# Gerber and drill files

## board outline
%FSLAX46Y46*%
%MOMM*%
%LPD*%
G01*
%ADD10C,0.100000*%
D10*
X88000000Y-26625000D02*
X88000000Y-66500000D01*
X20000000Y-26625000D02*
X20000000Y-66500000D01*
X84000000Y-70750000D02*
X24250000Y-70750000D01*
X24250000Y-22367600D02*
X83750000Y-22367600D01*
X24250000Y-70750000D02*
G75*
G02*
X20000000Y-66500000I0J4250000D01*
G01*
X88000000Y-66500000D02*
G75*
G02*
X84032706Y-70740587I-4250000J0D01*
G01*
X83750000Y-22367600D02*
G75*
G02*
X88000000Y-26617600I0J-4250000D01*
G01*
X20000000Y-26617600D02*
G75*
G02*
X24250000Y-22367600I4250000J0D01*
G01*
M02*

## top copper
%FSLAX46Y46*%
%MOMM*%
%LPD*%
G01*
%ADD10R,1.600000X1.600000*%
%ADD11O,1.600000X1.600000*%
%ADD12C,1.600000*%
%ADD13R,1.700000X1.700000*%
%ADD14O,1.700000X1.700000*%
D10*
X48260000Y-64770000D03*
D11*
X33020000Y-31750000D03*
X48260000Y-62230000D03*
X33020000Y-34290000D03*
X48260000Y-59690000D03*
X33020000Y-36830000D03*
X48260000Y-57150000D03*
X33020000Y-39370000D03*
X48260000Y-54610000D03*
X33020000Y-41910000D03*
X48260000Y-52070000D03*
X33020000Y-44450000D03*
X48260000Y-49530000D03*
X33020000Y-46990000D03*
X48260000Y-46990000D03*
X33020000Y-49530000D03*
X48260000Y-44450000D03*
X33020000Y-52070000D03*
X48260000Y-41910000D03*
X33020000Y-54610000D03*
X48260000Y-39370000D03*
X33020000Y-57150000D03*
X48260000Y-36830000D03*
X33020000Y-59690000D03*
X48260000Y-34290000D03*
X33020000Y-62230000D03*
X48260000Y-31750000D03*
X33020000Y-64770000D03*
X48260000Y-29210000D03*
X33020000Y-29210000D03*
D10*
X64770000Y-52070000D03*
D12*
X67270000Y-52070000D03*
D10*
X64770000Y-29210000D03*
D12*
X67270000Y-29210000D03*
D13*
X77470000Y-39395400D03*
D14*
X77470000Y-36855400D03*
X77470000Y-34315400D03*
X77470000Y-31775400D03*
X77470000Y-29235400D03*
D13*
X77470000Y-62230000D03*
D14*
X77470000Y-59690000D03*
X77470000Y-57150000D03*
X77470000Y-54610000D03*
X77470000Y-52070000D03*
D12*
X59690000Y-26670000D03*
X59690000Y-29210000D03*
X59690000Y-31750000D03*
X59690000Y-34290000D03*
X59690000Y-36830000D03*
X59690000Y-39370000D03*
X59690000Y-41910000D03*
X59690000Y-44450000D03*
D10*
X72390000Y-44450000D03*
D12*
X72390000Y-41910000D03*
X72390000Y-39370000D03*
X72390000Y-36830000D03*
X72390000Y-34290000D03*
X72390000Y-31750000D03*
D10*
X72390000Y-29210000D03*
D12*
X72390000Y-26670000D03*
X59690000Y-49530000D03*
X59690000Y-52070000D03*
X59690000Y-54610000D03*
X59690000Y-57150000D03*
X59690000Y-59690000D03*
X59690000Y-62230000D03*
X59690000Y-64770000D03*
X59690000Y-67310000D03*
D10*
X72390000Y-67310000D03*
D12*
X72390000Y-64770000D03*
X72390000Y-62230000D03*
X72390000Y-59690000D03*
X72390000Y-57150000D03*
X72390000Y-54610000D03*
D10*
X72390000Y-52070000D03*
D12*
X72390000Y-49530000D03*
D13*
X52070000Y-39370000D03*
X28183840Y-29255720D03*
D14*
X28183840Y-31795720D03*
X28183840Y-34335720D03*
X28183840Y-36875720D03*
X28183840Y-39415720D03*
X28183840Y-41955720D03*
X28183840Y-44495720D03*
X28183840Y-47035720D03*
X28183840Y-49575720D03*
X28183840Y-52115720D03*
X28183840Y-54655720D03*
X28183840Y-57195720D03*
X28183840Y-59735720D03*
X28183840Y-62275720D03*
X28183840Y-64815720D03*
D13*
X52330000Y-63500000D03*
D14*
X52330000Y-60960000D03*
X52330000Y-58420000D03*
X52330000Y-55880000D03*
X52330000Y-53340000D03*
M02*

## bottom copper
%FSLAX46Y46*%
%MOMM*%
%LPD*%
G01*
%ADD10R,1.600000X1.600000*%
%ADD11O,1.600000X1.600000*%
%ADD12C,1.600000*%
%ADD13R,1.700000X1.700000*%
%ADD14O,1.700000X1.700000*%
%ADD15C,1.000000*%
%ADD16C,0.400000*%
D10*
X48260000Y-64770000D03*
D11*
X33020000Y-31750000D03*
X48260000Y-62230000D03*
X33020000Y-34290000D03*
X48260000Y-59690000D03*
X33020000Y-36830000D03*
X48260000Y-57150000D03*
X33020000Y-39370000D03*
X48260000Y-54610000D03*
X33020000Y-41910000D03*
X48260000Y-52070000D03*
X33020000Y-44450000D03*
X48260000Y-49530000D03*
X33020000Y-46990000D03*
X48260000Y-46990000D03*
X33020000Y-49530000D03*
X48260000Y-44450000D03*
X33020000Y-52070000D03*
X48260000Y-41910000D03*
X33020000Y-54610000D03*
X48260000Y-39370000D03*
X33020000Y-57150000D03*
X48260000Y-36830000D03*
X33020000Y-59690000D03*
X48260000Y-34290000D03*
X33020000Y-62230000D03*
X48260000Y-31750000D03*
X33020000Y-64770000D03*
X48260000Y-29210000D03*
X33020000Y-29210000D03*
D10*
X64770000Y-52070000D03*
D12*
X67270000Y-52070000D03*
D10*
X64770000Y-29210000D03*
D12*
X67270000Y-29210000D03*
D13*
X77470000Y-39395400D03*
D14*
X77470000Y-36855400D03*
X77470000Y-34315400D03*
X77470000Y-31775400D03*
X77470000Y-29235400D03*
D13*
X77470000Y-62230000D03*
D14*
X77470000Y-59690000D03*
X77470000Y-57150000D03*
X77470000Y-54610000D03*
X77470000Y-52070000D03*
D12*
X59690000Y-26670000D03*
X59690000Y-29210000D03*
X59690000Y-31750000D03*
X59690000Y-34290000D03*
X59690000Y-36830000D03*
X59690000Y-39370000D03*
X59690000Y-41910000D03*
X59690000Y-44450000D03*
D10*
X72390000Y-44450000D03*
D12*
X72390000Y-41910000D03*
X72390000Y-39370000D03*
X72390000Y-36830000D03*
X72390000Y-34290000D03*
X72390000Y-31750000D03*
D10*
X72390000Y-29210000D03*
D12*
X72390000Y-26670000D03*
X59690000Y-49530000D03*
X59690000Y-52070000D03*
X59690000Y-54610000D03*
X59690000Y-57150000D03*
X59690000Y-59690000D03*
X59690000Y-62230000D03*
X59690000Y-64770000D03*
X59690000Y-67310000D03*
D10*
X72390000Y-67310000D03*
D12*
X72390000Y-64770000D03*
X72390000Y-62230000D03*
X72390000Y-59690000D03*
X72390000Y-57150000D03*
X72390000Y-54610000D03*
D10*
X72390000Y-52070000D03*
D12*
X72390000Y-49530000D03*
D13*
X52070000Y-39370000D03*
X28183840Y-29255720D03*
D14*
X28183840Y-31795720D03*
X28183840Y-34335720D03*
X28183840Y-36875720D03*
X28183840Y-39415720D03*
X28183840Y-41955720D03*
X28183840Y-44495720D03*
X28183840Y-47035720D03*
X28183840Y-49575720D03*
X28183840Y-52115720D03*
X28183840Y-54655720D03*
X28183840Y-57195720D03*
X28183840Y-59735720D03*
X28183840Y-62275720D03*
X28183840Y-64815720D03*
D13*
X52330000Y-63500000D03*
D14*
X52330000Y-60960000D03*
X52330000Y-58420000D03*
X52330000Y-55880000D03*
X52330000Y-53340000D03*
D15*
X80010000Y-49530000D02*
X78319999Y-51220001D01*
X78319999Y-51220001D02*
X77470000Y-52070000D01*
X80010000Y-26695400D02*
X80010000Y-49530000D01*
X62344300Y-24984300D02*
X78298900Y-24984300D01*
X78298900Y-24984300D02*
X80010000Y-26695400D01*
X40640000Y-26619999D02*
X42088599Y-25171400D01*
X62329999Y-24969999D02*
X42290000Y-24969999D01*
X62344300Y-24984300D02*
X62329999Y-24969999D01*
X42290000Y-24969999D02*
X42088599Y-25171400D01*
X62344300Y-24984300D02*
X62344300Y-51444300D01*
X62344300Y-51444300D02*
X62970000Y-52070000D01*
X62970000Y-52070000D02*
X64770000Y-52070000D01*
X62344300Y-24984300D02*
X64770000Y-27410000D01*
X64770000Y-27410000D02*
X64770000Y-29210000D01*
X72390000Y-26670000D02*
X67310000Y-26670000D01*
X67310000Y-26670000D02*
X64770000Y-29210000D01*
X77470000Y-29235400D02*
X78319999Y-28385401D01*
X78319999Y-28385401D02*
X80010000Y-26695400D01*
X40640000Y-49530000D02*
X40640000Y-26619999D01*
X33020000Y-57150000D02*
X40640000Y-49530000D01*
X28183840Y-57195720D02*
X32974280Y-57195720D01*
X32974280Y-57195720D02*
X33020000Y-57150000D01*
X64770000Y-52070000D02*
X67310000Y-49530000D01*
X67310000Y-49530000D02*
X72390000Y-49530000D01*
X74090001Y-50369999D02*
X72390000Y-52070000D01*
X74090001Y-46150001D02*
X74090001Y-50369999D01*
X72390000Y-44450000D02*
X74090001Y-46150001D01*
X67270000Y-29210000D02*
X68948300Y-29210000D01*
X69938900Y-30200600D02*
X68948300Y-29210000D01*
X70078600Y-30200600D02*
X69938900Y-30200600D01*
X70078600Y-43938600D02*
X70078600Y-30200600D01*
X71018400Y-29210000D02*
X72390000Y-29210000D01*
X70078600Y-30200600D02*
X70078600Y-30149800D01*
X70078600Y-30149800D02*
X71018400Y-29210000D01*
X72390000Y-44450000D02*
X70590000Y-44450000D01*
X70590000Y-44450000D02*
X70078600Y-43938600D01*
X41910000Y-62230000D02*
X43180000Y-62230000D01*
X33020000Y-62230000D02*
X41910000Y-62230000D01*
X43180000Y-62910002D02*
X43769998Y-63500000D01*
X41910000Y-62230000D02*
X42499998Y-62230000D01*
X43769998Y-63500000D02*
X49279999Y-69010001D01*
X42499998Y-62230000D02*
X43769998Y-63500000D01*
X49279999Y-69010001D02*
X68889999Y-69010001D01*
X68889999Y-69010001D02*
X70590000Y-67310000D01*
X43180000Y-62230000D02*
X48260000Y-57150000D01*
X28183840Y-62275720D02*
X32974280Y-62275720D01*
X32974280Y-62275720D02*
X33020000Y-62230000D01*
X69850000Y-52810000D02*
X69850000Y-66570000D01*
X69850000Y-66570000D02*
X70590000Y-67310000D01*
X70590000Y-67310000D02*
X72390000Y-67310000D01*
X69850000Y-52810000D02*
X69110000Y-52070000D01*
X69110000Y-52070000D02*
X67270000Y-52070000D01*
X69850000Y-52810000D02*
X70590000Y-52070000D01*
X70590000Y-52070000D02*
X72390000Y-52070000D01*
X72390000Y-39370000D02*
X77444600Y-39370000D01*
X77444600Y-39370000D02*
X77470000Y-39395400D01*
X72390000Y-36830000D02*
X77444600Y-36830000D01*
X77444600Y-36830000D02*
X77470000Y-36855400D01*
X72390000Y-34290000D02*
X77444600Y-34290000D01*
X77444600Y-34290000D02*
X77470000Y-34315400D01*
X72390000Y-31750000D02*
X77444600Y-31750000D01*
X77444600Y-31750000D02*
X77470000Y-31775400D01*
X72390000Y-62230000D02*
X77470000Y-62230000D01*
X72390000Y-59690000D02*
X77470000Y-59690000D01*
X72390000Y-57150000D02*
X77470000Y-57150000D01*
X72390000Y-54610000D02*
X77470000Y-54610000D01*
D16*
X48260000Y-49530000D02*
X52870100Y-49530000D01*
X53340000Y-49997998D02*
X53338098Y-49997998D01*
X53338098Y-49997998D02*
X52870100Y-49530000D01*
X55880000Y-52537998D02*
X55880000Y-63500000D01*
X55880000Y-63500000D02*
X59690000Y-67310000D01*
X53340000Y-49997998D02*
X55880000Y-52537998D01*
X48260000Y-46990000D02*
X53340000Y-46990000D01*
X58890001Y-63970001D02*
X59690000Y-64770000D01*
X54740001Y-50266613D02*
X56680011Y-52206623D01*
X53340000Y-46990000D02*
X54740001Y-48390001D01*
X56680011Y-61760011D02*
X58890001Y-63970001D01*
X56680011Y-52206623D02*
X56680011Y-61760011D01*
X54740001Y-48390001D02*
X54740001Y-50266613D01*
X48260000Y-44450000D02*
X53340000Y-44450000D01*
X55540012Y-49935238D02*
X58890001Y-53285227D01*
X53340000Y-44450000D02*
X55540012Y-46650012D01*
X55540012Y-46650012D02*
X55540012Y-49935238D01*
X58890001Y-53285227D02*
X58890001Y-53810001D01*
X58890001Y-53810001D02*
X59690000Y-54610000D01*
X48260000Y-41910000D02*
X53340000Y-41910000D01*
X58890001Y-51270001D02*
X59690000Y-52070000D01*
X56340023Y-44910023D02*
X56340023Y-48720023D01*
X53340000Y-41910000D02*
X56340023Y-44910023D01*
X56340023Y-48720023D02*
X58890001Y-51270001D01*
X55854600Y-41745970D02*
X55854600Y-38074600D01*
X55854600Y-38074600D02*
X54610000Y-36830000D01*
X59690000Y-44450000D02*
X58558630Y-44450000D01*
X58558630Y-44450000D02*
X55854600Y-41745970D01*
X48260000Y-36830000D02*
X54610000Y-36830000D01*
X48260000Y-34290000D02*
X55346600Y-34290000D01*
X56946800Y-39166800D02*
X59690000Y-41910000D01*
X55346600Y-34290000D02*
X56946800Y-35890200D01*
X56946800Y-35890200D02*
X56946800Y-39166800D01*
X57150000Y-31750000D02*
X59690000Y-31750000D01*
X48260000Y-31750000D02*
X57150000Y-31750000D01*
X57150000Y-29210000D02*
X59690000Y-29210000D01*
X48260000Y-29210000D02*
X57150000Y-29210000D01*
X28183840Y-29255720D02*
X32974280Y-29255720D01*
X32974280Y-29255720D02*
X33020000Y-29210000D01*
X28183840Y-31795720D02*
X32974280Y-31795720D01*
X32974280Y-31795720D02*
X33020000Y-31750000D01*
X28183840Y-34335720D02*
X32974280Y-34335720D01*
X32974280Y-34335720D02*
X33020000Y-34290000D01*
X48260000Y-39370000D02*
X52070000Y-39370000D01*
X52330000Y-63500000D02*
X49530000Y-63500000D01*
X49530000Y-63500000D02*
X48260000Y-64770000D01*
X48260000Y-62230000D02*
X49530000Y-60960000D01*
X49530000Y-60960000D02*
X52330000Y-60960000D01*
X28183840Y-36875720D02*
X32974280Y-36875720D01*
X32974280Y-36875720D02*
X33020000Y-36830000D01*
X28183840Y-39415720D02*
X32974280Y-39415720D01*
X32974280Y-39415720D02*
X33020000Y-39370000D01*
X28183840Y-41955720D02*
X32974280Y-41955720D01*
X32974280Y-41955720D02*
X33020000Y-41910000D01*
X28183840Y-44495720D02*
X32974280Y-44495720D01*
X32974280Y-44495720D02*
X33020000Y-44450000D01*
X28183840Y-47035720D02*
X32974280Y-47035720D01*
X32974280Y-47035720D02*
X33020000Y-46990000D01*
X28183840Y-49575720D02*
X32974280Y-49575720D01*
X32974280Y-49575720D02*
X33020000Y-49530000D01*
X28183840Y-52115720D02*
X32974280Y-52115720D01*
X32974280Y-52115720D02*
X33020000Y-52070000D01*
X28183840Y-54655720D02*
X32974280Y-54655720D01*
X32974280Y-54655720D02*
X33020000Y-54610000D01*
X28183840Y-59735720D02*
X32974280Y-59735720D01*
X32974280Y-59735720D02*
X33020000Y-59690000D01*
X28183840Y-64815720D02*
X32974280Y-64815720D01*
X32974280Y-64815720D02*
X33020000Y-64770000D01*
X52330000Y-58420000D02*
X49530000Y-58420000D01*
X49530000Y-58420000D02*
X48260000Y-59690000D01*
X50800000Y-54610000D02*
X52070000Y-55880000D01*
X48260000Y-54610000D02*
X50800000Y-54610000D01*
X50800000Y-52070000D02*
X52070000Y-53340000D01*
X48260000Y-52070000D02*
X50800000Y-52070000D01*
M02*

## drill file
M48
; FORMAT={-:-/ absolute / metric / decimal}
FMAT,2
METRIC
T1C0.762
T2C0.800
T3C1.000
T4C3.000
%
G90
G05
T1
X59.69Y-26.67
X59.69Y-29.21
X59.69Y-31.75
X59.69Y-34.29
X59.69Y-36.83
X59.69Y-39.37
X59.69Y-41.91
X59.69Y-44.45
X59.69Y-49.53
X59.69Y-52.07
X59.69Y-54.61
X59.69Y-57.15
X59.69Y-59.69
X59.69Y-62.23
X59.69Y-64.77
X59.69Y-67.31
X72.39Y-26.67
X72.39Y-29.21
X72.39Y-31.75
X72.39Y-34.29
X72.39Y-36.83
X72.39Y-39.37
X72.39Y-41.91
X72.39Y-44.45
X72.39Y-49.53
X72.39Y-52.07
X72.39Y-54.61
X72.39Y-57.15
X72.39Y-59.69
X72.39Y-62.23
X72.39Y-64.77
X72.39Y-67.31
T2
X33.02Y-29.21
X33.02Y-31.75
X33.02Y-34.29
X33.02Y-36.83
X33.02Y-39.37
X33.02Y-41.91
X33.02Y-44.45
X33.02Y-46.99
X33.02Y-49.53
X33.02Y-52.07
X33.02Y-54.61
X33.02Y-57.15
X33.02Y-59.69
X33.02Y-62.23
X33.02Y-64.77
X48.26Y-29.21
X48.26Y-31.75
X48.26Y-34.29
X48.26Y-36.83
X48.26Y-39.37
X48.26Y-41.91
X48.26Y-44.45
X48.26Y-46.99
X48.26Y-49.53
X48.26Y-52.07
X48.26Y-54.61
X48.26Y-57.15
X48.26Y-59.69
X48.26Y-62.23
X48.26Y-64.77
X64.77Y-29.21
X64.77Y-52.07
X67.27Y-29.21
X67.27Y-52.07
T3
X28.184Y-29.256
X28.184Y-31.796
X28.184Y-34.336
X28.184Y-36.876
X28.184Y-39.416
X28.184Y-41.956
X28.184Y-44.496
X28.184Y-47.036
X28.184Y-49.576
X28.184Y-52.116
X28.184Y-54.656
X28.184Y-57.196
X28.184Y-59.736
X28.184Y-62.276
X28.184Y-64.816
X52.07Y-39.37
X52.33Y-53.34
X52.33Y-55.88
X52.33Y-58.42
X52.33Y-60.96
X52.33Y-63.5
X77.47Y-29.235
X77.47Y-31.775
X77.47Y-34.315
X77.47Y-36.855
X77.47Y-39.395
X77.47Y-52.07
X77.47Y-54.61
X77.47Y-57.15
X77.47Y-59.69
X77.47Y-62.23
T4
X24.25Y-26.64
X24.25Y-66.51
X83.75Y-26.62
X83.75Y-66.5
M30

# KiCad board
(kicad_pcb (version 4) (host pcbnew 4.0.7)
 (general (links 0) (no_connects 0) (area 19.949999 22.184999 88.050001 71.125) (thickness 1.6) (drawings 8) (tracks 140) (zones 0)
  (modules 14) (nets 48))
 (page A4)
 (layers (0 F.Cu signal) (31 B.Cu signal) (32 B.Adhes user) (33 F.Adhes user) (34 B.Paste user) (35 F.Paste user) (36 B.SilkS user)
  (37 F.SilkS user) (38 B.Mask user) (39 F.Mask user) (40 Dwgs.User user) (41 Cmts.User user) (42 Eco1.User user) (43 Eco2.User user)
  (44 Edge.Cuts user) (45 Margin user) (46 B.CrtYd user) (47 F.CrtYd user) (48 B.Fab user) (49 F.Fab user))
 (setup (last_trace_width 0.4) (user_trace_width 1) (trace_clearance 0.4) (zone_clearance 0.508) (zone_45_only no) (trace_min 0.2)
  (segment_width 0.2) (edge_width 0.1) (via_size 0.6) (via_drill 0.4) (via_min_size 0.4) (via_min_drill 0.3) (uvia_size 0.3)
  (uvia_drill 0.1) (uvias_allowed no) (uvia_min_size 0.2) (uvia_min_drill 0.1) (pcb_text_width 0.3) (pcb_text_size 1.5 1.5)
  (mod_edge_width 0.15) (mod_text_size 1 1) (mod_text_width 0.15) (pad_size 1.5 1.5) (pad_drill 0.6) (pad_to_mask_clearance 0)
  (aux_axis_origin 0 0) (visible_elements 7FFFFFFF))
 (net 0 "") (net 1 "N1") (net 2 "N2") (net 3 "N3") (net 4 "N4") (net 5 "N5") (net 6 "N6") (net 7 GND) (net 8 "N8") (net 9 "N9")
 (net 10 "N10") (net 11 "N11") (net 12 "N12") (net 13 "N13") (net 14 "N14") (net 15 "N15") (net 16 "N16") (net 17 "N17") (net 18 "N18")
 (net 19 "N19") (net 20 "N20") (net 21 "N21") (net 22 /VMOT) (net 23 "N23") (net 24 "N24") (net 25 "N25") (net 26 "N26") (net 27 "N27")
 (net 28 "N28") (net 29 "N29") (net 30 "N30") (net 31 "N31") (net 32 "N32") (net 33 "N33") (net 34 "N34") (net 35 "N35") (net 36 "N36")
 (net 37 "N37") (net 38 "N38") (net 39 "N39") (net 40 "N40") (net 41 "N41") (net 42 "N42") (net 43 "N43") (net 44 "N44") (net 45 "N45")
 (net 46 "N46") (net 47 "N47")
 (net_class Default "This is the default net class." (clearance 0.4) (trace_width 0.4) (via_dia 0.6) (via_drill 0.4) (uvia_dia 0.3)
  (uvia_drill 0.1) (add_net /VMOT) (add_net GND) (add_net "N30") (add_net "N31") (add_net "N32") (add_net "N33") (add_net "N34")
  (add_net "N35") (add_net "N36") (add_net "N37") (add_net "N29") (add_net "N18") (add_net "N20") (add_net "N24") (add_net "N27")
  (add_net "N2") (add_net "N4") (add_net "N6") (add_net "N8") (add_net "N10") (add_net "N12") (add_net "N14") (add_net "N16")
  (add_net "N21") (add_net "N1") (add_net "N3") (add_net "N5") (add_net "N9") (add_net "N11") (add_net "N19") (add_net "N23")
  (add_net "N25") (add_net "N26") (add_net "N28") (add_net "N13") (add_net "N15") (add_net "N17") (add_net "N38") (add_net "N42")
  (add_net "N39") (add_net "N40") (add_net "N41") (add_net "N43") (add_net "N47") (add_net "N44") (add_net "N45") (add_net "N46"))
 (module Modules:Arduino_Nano (layer F.Cu) (at 48.26 64.77 180)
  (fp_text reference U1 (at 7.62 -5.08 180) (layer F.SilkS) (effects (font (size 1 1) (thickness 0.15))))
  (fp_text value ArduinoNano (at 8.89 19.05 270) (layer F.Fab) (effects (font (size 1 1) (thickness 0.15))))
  (pad 1 thru_hole rect (at 0 0 180) (size 1.6 1.6) (drill 0.8) (layers *.Cu *.Mask) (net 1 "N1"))
  (pad 17 thru_hole oval (at 15.24 33.02 180) (size 1.6 1.6) (drill 0.8) (layers *.Cu *.Mask) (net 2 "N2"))
  (pad 2 thru_hole oval (at 0 2.54 180) (size 1.6 1.6) (drill 0.8) (layers *.Cu *.Mask) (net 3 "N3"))
  (pad 18 thru_hole oval (at 15.24 30.48 180) (size 1.6 1.6) (drill 0.8) (layers *.Cu *.Mask) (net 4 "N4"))
  (pad 3 thru_hole oval (at 0 5.08 180) (size 1.6 1.6) (drill 0.8) (layers *.Cu *.Mask) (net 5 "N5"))
  (pad 19 thru_hole oval (at 15.24 27.94 180) (size 1.6 1.6) (drill 0.8) (layers *.Cu *.Mask) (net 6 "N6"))
  (pad 4 thru_hole oval (at 0 7.62 180) (size 1.6 1.6) (drill 0.8) (layers *.Cu *.Mask) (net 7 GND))
  (pad 20 thru_hole oval (at 15.24 25.4 180) (size 1.6 1.6) (drill 0.8) (layers *.Cu *.Mask) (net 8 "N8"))
  (pad 5 thru_hole oval (at 0 10.16 180) (size 1.6 1.6) (drill 0.8) (layers *.Cu *.Mask) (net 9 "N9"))
  (pad 21 thru_hole oval (at 15.24 22.86 180) (size 1.6 1.6) (drill 0.8) (layers *.Cu *.Mask) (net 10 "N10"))
  (pad 6 thru_hole oval (at 0 12.7 180) (size 1.6 1.6) (drill 0.8) (layers *.Cu *.Mask) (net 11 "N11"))
  (pad 22 thru_hole oval (at 15.24 20.32 180) (size 1.6 1.6) (drill 0.8) (layers *.Cu *.Mask) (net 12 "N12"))
  (pad 7 thru_hole oval (at 0 15.24 180) (size 1.6 1.6) (drill 0.8) (layers *.Cu *.Mask) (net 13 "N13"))
  (pad 23 thru_hole oval (at 15.24 17.78 180) (size 1.6 1.6) (drill 0.8) (layers *.Cu *.Mask) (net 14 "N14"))
  (pad 8 thru_hole oval (at 0 17.78 180) (size 1.6 1.6) (drill 0.8) (layers *.Cu *.Mask) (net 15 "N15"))
  (pad 24 thru_hole oval (at 15.24 15.24 180) (size 1.6 1.6) (drill 0.8) (layers *.Cu *.Mask) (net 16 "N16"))
  (pad 9 thru_hole oval (at 0 20.32 180) (size 1.6 1.6) (drill 0.8) (layers *.Cu *.Mask) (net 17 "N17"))
  (pad 25 thru_hole oval (at 15.24 12.7 180) (size 1.6 1.6) (drill 0.8) (layers *.Cu *.Mask) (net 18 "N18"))
  (pad 10 thru_hole oval (at 0 22.86 180) (size 1.6 1.6) (drill 0.8) (layers *.Cu *.Mask) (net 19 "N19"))
  (pad 26 thru_hole oval (at 15.24 10.16 180) (size 1.6 1.6) (drill 0.8) (layers *.Cu *.Mask) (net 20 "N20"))
  (pad 11 thru_hole oval (at 0 25.4 180) (size 1.6 1.6) (drill 0.8) (layers *.Cu *.Mask) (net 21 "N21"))
  (pad 27 thru_hole oval (at 15.24 7.62 180) (size 1.6 1.6) (drill 0.8) (layers *.Cu *.Mask) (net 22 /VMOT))
  (pad 12 thru_hole oval (at 0 27.94 180) (size 1.6 1.6) (drill 0.8) (layers *.Cu *.Mask) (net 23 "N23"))
  (pad 28 thru_hole oval (at 15.24 5.08 180) (size 1.6 1.6) (drill 0.8) (layers *.Cu *.Mask) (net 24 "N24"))
  (pad 13 thru_hole oval (at 0 30.48 180) (size 1.6 1.6) (drill 0.8) (layers *.Cu *.Mask) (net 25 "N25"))
  (pad 29 thru_hole oval (at 15.24 2.54 180) (size 1.6 1.6) (drill 0.8) (layers *.Cu *.Mask) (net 7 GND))
  (pad 14 thru_hole oval (at 0 33.02 180) (size 1.6 1.6) (drill 0.8) (layers *.Cu *.Mask) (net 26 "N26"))
  (pad 30 thru_hole oval (at 15.24 0 180) (size 1.6 1.6) (drill 0.8) (layers *.Cu *.Mask) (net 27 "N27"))
  (pad 15 thru_hole oval (at 0 35.56 180) (size 1.6 1.6) (drill 0.8) (layers *.Cu *.Mask) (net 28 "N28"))
  (pad 16 thru_hole oval (at 15.24 35.56 180) (size 1.6 1.6) (drill 0.8) (layers *.Cu *.Mask) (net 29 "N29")))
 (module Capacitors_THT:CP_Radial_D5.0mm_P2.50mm (layer F.Cu) (at 64.77 52.07)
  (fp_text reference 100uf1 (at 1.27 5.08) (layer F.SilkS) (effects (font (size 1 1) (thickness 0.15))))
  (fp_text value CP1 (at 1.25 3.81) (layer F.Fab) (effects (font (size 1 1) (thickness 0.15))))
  (pad 1 thru_hole rect (at 0 0) (size 1.6 1.6) (drill 0.8) (layers *.Cu *.Mask) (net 22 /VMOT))
  (pad 2 thru_hole circle (at 2.5 0) (size 1.6 1.6) (drill 0.8) (layers *.Cu *.Mask) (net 7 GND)))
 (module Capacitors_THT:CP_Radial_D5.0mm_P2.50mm (layer F.Cu) (at 64.77 29.21)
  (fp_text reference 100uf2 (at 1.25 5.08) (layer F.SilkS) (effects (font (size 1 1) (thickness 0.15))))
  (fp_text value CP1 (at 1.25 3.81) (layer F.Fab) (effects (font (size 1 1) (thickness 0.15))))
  (pad 1 thru_hole rect (at 0 0) (size 1.6 1.6) (drill 0.8) (layers *.Cu *.Mask) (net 22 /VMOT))
  (pad 2 thru_hole circle (at 2.5 0) (size 1.6 1.6) (drill 0.8) (layers *.Cu *.Mask) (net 7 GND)))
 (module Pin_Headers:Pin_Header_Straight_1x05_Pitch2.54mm (layer F.Cu) (at 77.47 39.3954 180)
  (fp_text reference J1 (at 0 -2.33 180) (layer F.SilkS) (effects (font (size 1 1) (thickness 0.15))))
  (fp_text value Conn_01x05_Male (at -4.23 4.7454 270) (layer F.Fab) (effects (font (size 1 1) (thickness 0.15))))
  (pad 1 thru_hole rect (at 0 0 180) (size 1.7 1.7) (drill 1) (layers *.Cu *.Mask) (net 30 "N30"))
  (pad 2 thru_hole oval (at 0 2.54 180) (size 1.7 1.7) (drill 1) (layers *.Cu *.Mask) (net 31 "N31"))
  (pad 3 thru_hole oval (at 0 5.08 180) (size 1.7 1.7) (drill 1) (layers *.Cu *.Mask) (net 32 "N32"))
  (pad 4 thru_hole oval (at 0 7.62 180) (size 1.7 1.7) (drill 1) (layers *.Cu *.Mask) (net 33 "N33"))
  (pad 5 thru_hole oval (at 0 10.16 180) (size 1.7 1.7) (drill 1) (layers *.Cu *.Mask) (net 22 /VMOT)))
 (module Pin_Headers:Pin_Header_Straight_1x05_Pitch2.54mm (layer F.Cu) (at 77.47 62.23 180)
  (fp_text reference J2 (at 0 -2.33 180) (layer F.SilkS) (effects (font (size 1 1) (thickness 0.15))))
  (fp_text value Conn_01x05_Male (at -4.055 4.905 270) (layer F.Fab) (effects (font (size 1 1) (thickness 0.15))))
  (pad 1 thru_hole rect (at 0 0 180) (size 1.7 1.7) (drill 1) (layers *.Cu *.Mask) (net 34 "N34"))
  (pad 2 thru_hole oval (at 0 2.54 180) (size 1.7 1.7) (drill 1) (layers *.Cu *.Mask) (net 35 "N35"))
  (pad 3 thru_hole oval (at 0 5.08 180) (size 1.7 1.7) (drill 1) (layers *.Cu *.Mask) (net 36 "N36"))
  (pad 4 thru_hole oval (at 0 7.62 180) (size 1.7 1.7) (drill 1) (layers *.Cu *.Mask) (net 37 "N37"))
  (pad 5 thru_hole oval (at 0 10.16 180) (size 1.7 1.7) (drill 1) (layers *.Cu *.Mask) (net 22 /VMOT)))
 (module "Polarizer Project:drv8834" (layer F.Cu) (at 59.69 26.67)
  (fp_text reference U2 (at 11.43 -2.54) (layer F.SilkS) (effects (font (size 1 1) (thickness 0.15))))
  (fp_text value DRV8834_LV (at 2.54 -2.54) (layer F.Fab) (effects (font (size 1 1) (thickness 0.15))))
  (pad 1 thru_hole circle (at 0 0) (size 1.6 1.6) (drill 0.762) (layers *.Cu *.Mask) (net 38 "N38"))
  (pad 2 thru_hole circle (at 0 2.54) (size 1.6 1.6) (drill 0.762) (layers *.Cu *.Mask) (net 28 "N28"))
  (pad 3 thru_hole circle (at 0 5.08) (size 1.6 1.6) (drill 0.762) (layers *.Cu *.Mask) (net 26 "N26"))
  (pad 4 thru_hole circle (at 0 7.62) (size 1.6 1.6) (drill 0.762) (layers *.Cu *.Mask) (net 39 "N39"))
  (pad 5 thru_hole circle (at 0 10.16) (size 1.6 1.6) (drill 0.762) (layers *.Cu *.Mask) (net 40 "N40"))
  (pad 6 thru_hole circle (at 0 12.7) (size 1.6 1.6) (drill 0.762) (layers *.Cu *.Mask) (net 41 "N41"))
  (pad 7 thru_hole circle (at 0 15.24) (size 1.6 1.6) (drill 0.762) (layers *.Cu *.Mask) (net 25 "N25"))
  (pad 8 thru_hole circle (at 0 17.78) (size 1.6 1.6) (drill 0.762) (layers *.Cu *.Mask) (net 23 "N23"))
  (pad 9 thru_hole rect (at 12.7 17.78) (size 1.6 1.6) (drill 0.762) (layers *.Cu *.Mask) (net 7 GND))
  (pad 10 thru_hole circle (at 12.7 15.24) (size 1.6 1.6) (drill 0.762) (layers *.Cu *.Mask) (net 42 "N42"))
  (pad 11 thru_hole circle (at 12.7 12.7) (size 1.6 1.6) (drill 0.762) (layers *.Cu *.Mask) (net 30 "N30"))
  (pad 12 thru_hole circle (at 12.7 10.16) (size 1.6 1.6) (drill 0.762) (layers *.Cu *.Mask) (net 31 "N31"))
  (pad 13 thru_hole circle (at 12.7 7.62) (size 1.6 1.6) (drill 0.762) (layers *.Cu *.Mask) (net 32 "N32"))
  (pad 14 thru_hole circle (at 12.7 5.08) (size 1.6 1.6) (drill 0.762) (layers *.Cu *.Mask) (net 33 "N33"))
  (pad 15 thru_hole rect (at 12.7 2.54) (size 1.6 1.6) (drill 0.762) (layers *.Cu *.Mask) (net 7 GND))
  (pad 16 thru_hole circle (at 12.7 0) (size 1.6 1.6) (drill 0.762) (layers *.Cu *.Mask) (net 22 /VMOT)))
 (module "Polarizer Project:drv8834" (layer F.Cu) (at 59.69 49.53)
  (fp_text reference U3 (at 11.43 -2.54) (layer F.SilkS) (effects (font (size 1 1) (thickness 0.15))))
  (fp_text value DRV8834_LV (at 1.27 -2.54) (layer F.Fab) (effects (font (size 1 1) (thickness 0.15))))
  (pad 1 thru_hole circle (at 0 0) (size 1.6 1.6) (drill 0.762) (layers *.Cu *.Mask) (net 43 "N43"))
  (pad 2 thru_hole circle (at 0 2.54) (size 1.6 1.6) (drill 0.762) (layers *.Cu *.Mask) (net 19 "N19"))
  (pad 3 thru_hole circle (at 0 5.08) (size 1.6 1.6) (drill 0.762) (layers *.Cu *.Mask) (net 17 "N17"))
  (pad 4 thru_hole circle (at 0 7.62) (size 1.6 1.6) (drill 0.762) (layers *.Cu *.Mask) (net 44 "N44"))
  (pad 5 thru_hole circle (at 0 10.16) (size 1.6 1.6) (drill 0.762) (layers *.Cu *.Mask) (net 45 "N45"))
  (pad 6 thru_hole circle (at 0 12.7) (size 1.6 1.6) (drill 0.762) (layers *.Cu *.Mask) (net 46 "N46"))
  (pad 7 thru_hole circle (at 0 15.24) (size 1.6 1.6) (drill 0.762) (layers *.Cu *.Mask) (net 15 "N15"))
  (pad 8 thru_hole circle (at 0 17.78) (size 1.6 1.6) (drill 0.762) (layers *.Cu *.Mask) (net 13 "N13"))
  (pad 9 thru_hole rect (at 12.7 17.78) (size 1.6 1.6) (drill 0.762) (layers *.Cu *.Mask) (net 7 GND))
  (pad 10 thru_hole circle (at 12.7 15.24) (size 1.6 1.6) (drill 0.762) (layers *.Cu *.Mask) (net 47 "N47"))
  (pad 11 thru_hole circle (at 12.7 12.7) (size 1.6 1.6) (drill 0.762) (layers *.Cu *.Mask) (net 34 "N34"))
  (pad 12 thru_hole circle (at 12.7 10.16) (size 1.6 1.6) (drill 0.762) (layers *.Cu *.Mask) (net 35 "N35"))
  (pad 13 thru_hole circle (at 12.7 7.62) (size 1.6 1.6) (drill 0.762) (layers *.Cu *.Mask) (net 36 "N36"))
  (pad 14 thru_hole circle (at 12.7 5.08) (size 1.6 1.6) (drill 0.762) (layers *.Cu *.Mask) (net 37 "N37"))
  (pad 15 thru_hole rect (at 12.7 2.54) (size 1.6 1.6) (drill 0.762) (layers *.Cu *.Mask) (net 7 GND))
  (pad 16 thru_hole circle (at 12.7 0) (size 1.6 1.6) (drill 0.762) (layers *.Cu *.Mask) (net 22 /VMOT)))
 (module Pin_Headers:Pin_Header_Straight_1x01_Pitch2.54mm (layer F.Cu) (at 52.07 39.37)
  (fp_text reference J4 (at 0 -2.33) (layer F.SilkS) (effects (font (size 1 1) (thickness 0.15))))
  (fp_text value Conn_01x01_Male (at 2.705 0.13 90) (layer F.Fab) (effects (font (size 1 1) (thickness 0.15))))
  (pad 1 thru_hole rect (at 0 0) (size 1.7 1.7) (drill 1) (layers *.Cu *.Mask) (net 21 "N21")))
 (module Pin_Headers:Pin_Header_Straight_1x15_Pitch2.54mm (layer F.Cu) (at 28.18384 29.25572)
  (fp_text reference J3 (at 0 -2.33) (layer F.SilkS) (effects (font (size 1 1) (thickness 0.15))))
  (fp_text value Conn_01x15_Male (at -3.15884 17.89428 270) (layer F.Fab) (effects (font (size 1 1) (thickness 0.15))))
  (pad 1 thru_hole rect (at 0 0) (size 1.7 1.7) (drill 1) (layers *.Cu *.Mask) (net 29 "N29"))
  (pad 2 thru_hole oval (at 0 2.54) (size 1.7 1.7) (drill 1) (layers *.Cu *.Mask) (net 2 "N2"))
  (pad 3 thru_hole oval (at 0 5.08) (size 1.7 1.7) (drill 1) (layers *.Cu *.Mask) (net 4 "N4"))
  (pad 4 thru_hole oval (at 0 7.62) (size 1.7 1.7) (drill 1) (layers *.Cu *.Mask) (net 6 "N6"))
  (pad 5 thru_hole oval (at 0 10.16) (size 1.7 1.7) (drill 1) (layers *.Cu *.Mask) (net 8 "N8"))
  (pad 6 thru_hole oval (at 0 12.7) (size 1.7 1.7) (drill 1) (layers *.Cu *.Mask) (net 10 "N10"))
  (pad 7 thru_hole oval (at 0 15.24) (size 1.7 1.7) (drill 1) (layers *.Cu *.Mask) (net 12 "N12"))
  (pad 8 thru_hole oval (at 0 17.78) (size 1.7 1.7) (drill 1) (layers *.Cu *.Mask) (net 14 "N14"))
  (pad 9 thru_hole oval (at 0 20.32) (size 1.7 1.7) (drill 1) (layers *.Cu *.Mask) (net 16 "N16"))
  (pad 10 thru_hole oval (at 0 22.86) (size 1.7 1.7) (drill 1) (layers *.Cu *.Mask) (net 18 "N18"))
  (pad 11 thru_hole oval (at 0 25.4) (size 1.7 1.7) (drill 1) (layers *.Cu *.Mask) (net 20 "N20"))
  (pad 12 thru_hole oval (at 0 27.94) (size 1.7 1.7) (drill 1) (layers *.Cu *.Mask) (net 22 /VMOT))
  (pad 13 thru_hole oval (at 0 30.48) (size 1.7 1.7) (drill 1) (layers *.Cu *.Mask) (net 24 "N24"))
  (pad 14 thru_hole oval (at 0 33.02) (size 1.7 1.7) (drill 1) (layers *.Cu *.Mask) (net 7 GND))
  (pad 15 thru_hole oval (at 0 35.56) (size 1.7 1.7) (drill 1) (layers *.Cu *.Mask) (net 27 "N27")))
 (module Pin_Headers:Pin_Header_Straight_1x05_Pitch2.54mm (layer F.Cu) (at 52.33 63.5 180)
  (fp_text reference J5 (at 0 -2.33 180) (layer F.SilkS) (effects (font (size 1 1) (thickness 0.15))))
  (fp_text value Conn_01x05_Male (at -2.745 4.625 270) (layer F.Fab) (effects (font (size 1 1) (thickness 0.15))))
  (pad 1 thru_hole rect (at 0 0 180) (size 1.7 1.7) (drill 1) (layers *.Cu *.Mask) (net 1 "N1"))
  (pad 2 thru_hole oval (at 0 2.54 180) (size 1.7 1.7) (drill 1) (layers *.Cu *.Mask) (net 3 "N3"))
  (pad 3 thru_hole oval (at 0 5.08 180) (size 1.7 1.7) (drill 1) (layers *.Cu *.Mask) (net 5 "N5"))
  (pad 4 thru_hole oval (at 0 7.62 180) (size 1.7 1.7) (drill 1) (layers *.Cu *.Mask) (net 9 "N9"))
  (pad 5 thru_hole oval (at 0 10.16 180) (size 1.7 1.7) (drill 1) (layers *.Cu *.Mask) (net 11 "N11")))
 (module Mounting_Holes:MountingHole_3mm (layer F.Cu) (at 24.25 26.64)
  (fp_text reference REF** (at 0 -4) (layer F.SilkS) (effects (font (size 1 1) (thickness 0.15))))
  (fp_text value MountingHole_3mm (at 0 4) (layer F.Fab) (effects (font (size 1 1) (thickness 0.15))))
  (pad 1 np_thru_hole circle (at 0 0) (size 3 3) (drill 3) (layers *.Cu *.Mask)))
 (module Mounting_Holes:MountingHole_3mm (layer F.Cu) (at 24.25 66.51)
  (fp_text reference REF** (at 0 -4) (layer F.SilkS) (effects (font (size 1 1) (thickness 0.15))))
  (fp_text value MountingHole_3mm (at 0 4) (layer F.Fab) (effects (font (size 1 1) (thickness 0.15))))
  (pad 1 np_thru_hole circle (at 0 0) (size 3 3) (drill 3) (layers *.Cu *.Mask)))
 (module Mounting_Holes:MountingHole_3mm (layer F.Cu) (at 83.75 66.5)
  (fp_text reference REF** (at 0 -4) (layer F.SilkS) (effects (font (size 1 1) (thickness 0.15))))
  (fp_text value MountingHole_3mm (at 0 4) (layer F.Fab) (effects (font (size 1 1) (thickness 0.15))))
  (pad 1 np_thru_hole circle (at 0 0) (size 3 3) (drill 3) (layers *.Cu *.Mask)))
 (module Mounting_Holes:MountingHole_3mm (layer F.Cu) (at 83.75 26.62)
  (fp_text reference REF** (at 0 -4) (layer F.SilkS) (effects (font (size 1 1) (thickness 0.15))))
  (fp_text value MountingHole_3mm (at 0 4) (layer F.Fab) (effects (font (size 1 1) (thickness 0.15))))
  (pad 1 np_thru_hole circle (at 0 0) (size 3 3) (drill 3) (layers *.Cu *.Mask)))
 (gr_line (start 88 26.625) (end 88 66.5) (layer Edge.Cuts) (width 0.1))
 (gr_line (start 20 26.625) (end 20 66.5) (layer Edge.Cuts) (width 0.1))
 (gr_line (start 84 70.75) (end 24.25 70.75) (layer Edge.Cuts) (width 0.1))
 (gr_line (start 24.25 22.3676) (end 83.75 22.3676) (layer Edge.Cuts) (width 0.1))
 (gr_arc (start 24.25 66.5) (end 24.25 70.75) (angle 90) (layer Edge.Cuts) (width 0.1))
 (gr_arc (start 83.75 66.5) (end 88 66.5) (angle 86.18592517) (layer Edge.Cuts) (width 0.1))
 (gr_arc (start 83.75 26.6176) (end 83.75 22.3676) (angle 90) (layer Edge.Cuts) (width 0.1))
 (gr_arc (start 24.25 26.6176) (end 20 26.6176) (angle 90) (layer Edge.Cuts) (width 0.1))
 (segment (start 80.01 49.53) (end 78.319999 51.220001) (width 1) (layer B.Cu) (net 22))
 (segment (start 78.319999 51.220001) (end 77.47 52.07) (width 1) (layer B.Cu) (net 22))
 (segment (start 80.01 26.6954) (end 80.01 49.53) (width 1) (layer B.Cu) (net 22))
 (segment (start 62.3443 24.9843) (end 78.2989 24.9843) (width 1) (layer B.Cu) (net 22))
 (segment (start 78.2989 24.9843) (end 80.01 26.6954) (width 1) (layer B.Cu) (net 22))
 (segment (start 40.64 26.619999) (end 42.088599 25.1714) (width 1) (layer B.Cu) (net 22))
 (segment (start 62.329999 24.969999) (end 42.29 24.969999) (width 1) (layer B.Cu) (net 22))
 (segment (start 62.3443 24.9843) (end 62.329999 24.969999) (width 1) (layer B.Cu) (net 22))
 (segment (start 42.29 24.969999) (end 42.088599 25.1714) (width 1) (layer B.Cu) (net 22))
 (segment (start 62.3443 24.9843) (end 62.3443 51.4443) (width 1) (layer B.Cu) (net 22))
 (segment (start 62.3443 51.4443) (end 62.97 52.07) (width 1) (layer B.Cu) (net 22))
 (segment (start 62.97 52.07) (end 64.77 52.07) (width 1) (layer B.Cu) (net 22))
 (segment (start 62.3443 24.9843) (end 64.77 27.41) (width 1) (layer B.Cu) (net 22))
 (segment (start 64.77 27.41) (end 64.77 29.21) (width 1) (layer B.Cu) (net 22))
 (segment (start 72.39 26.67) (end 67.31 26.67) (width 1) (layer B.Cu) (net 22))
 (segment (start 67.31 26.67) (end 64.77 29.21) (width 1) (layer B.Cu) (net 22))
 (segment (start 77.47 29.2354) (end 78.319999 28.385401) (width 1) (layer B.Cu) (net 22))
 (segment (start 78.319999 28.385401) (end 80.01 26.6954) (width 1) (layer B.Cu) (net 22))
 (segment (start 40.64 49.53) (end 40.64 26.619999) (width 1) (layer B.Cu) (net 22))
 (segment (start 33.02 57.15) (end 40.64 49.53) (width 1) (layer B.Cu) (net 22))
 (segment (start 28.18384 57.19572) (end 32.97428 57.19572) (width 1) (layer B.Cu) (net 22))
 (segment (start 32.97428 57.19572) (end 33.02 57.15) (width 1) (layer B.Cu) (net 22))
 (segment (start 64.77 52.07) (end 67.31 49.53) (width 1) (layer B.Cu) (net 22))
 (segment (start 67.31 49.53) (end 72.39 49.53) (width 1) (layer B.Cu) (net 22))
 (segment (start 74.090001 50.369999) (end 72.39 52.07) (width 1) (layer B.Cu) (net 7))
 (segment (start 74.090001 46.150001) (end 74.090001 50.369999) (width 1) (layer B.Cu) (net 7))
 (segment (start 72.39 44.45) (end 74.090001 46.150001) (width 1) (layer B.Cu) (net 7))
 (segment (start 67.27 29.21) (end 68.9483 29.21) (width 1) (layer B.Cu) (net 7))
 (segment (start 69.9389 30.2006) (end 68.9483 29.21) (width 1) (layer B.Cu) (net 7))
 (segment (start 70.0786 30.2006) (end 69.9389 30.2006) (width 1) (layer B.Cu) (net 7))
 (segment (start 70.0786 43.9386) (end 70.0786 30.2006) (width 1) (layer B.Cu) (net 7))
 (segment (start 71.0184 29.21) (end 72.39 29.21) (width 1) (layer B.Cu) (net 7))
 (segment (start 70.0786 30.2006) (end 70.0786 30.1498) (width 1) (layer B.Cu) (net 7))
 (segment (start 70.0786 30.1498) (end 71.0184 29.21) (width 1) (layer B.Cu) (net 7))
 (segment (start 72.39 44.45) (end 70.59 44.45) (width 1) (layer B.Cu) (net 7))
 (segment (start 70.59 44.45) (end 70.0786 43.9386) (width 1) (layer B.Cu) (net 7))
 (segment (start 41.91 62.23) (end 43.18 62.23) (width 1) (layer B.Cu) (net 7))
 (segment (start 33.02 62.23) (end 41.91 62.23) (width 1) (layer B.Cu) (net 7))
 (segment (start 43.18 62.910002) (end 43.769998 63.5) (width 1) (layer B.Cu) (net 7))
 (segment (start 41.91 62.23) (end 42.499998 62.23) (width 1) (layer B.Cu) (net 7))
 (segment (start 43.769998 63.5) (end 49.279999 69.010001) (width 1) (layer B.Cu) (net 7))
 (segment (start 42.499998 62.23) (end 43.769998 63.5) (width 1) (layer B.Cu) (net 7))
 (segment (start 49.279999 69.010001) (end 68.889999 69.010001) (width 1) (layer B.Cu) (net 7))
 (segment (start 68.889999 69.010001) (end 70.59 67.31) (width 1) (layer B.Cu) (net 7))
 (segment (start 43.18 62.23) (end 48.26 57.15) (width 1) (layer B.Cu) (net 7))
 (segment (start 28.18384 62.27572) (end 32.97428 62.27572) (width 1) (layer B.Cu) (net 7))
 (segment (start 32.97428 62.27572) (end 33.02 62.23) (width 1) (layer B.Cu) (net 7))
 (segment (start 69.85 52.81) (end 69.85 66.57) (width 1) (layer B.Cu) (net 7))
 (segment (start 69.85 66.57) (end 70.59 67.31) (width 1) (layer B.Cu) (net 7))
 (segment (start 70.59 67.31) (end 72.39 67.31) (width 1) (layer B.Cu) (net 7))
 (segment (start 69.85 52.81) (end 69.11 52.07) (width 1) (layer B.Cu) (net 7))
 (segment (start 69.11 52.07) (end 67.27 52.07) (width 1) (layer B.Cu) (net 7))
 (segment (start 69.85 52.81) (end 70.59 52.07) (width 1) (layer B.Cu) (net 7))
 (segment (start 70.59 52.07) (end 72.39 52.07) (width 1) (layer B.Cu) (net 7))
 (segment (start 72.39 39.37) (end 77.4446 39.37) (width 1) (layer B.Cu) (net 30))
 (segment (start 77.4446 39.37) (end 77.47 39.3954) (width 1) (layer B.Cu) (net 30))
 (segment (start 72.39 36.83) (end 77.4446 36.83) (width 1) (layer B.Cu) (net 31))
 (segment (start 77.4446 36.83) (end 77.47 36.8554) (width 1) (layer B.Cu) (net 31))
 (segment (start 72.39 34.29) (end 77.4446 34.29) (width 1) (layer B.Cu) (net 32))
 (segment (start 77.4446 34.29) (end 77.47 34.3154) (width 1) (layer B.Cu) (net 32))
 (segment (start 72.39 31.75) (end 77.4446 31.75) (width 1) (layer B.Cu) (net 33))
 (segment (start 77.4446 31.75) (end 77.47 31.7754) (width 1) (layer B.Cu) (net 33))
 (segment (start 72.39 62.23) (end 77.47 62.23) (width 1) (layer B.Cu) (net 34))
 (segment (start 72.39 59.69) (end 77.47 59.69) (width 1) (layer B.Cu) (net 35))
 (segment (start 72.39 57.15) (end 77.47 57.15) (width 1) (layer B.Cu) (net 36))
 (segment (start 72.39 54.61) (end 77.47 54.61) (width 1) (layer B.Cu) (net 37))
 (segment (start 48.26 49.53) (end 52.8701 49.53) (width 0.4) (layer B.Cu) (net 13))
 (segment (start 53.34 49.997998) (end 53.338098 49.997998) (width 0.4) (layer B.Cu) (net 13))
 (segment (start 53.338098 49.997998) (end 52.8701 49.53) (width 0.4) (layer B.Cu) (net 13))
 (segment (start 55.88 52.537998) (end 55.88 63.5) (width 0.4) (layer B.Cu) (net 13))
 (segment (start 55.88 63.5) (end 59.69 67.31) (width 0.4) (layer B.Cu) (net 13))
 (segment (start 53.34 49.997998) (end 55.88 52.537998) (width 0.4) (layer B.Cu) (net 13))
 (segment (start 48.26 46.99) (end 53.34 46.99) (width 0.4) (layer B.Cu) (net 15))
 (segment (start 58.890001 63.970001) (end 59.69 64.77) (width 0.4) (layer B.Cu) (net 15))
 (segment (start 54.740001 50.266613) (end 56.680011 52.206623) (width 0.4) (layer B.Cu) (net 15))
 (segment (start 53.34 46.99) (end 54.740001 48.390001) (width 0.4) (layer B.Cu) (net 15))
 (segment (start 56.680011 61.760011) (end 58.890001 63.970001) (width 0.4) (layer B.Cu) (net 15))
 (segment (start 56.680011 52.206623) (end 56.680011 61.760011) (width 0.4) (layer B.Cu) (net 15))
 (segment (start 54.740001 48.390001) (end 54.740001 50.266613) (width 0.4) (layer B.Cu) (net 15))
 (segment (start 48.26 44.45) (end 53.34 44.45) (width 0.4) (layer B.Cu) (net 17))
 (segment (start 55.540012 49.935238) (end 58.890001 53.285227) (width 0.4) (layer B.Cu) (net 17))
 (segment (start 53.34 44.45) (end 55.540012 46.650012) (width 0.4) (layer B.Cu) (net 17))
 (segment (start 55.540012 46.650012) (end 55.540012 49.935238) (width 0.4) (layer B.Cu) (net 17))
 (segment (start 58.890001 53.285227) (end 58.890001 53.810001) (width 0.4) (layer B.Cu) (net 17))
 (segment (start 58.890001 53.810001) (end 59.69 54.61) (width 0.4) (layer B.Cu) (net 17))
 (segment (start 48.26 41.91) (end 53.34 41.91) (width 0.4) (layer B.Cu) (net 19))
 (segment (start 58.890001 51.270001) (end 59.69 52.07) (width 0.4) (layer B.Cu) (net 19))
 (segment (start 56.340023 44.910023) (end 56.340023 48.720023) (width 0.4) (layer B.Cu) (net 19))
 (segment (start 53.34 41.91) (end 56.340023 44.910023) (width 0.4) (layer B.Cu) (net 19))
 (segment (start 56.340023 48.720023) (end 58.890001 51.270001) (width 0.4) (layer B.Cu) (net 19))
 (segment (start 55.8546 41.74597) (end 55.8546 38.0746) (width 0.4) (layer B.Cu) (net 23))
 (segment (start 55.8546 38.0746) (end 54.61 36.83) (width 0.4) (layer B.Cu) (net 23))
 (segment (start 59.69 44.45) (end 58.55863 44.45) (width 0.4) (layer B.Cu) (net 23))
 (segment (start 58.55863 44.45) (end 55.8546 41.74597) (width 0.4) (layer B.Cu) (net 23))
 (segment (start 48.26 36.83) (end 54.61 36.83) (width 0.4) (layer B.Cu) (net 23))
 (segment (start 48.26 34.29) (end 55.3466 34.29) (width 0.4) (layer B.Cu) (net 25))
 (segment (start 56.9468 39.1668) (end 59.69 41.91) (width 0.4) (layer B.Cu) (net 25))
 (segment (start 55.3466 34.29) (end 56.9468 35.8902) (width 0.4) (layer B.Cu) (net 25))
 (segment (start 56.9468 35.8902) (end 56.9468 39.1668) (width 0.4) (layer B.Cu) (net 25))
 (segment (start 57.15 31.75) (end 59.69 31.75) (width 0.4) (layer B.Cu) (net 26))
 (segment (start 48.26 31.75) (end 57.15 31.75) (width 0.4) (layer B.Cu) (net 26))
 (segment (start 57.15 29.21) (end 59.69 29.21) (width 0.4) (layer B.Cu) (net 28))
 (segment (start 48.26 29.21) (end 57.15 29.21) (width 0.4) (layer B.Cu) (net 28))
 (segment (start 28.18384 29.25572) (end 32.97428 29.25572) (width 0.4) (layer B.Cu) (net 29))
 (segment (start 32.97428 29.25572) (end 33.02 29.21) (width 0.4) (layer B.Cu) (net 29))
 (segment (start 28.18384 31.79572) (end 32.97428 31.79572) (width 0.4) (layer B.Cu) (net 2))
 (segment (start 32.97428 31.79572) (end 33.02 31.75) (width 0.4) (layer B.Cu) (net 2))
 (segment (start 28.18384 34.33572) (end 32.97428 34.33572) (width 0.4) (layer B.Cu) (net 4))
 (segment (start 32.97428 34.33572) (end 33.02 34.29) (width 0.4) (layer B.Cu) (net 4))
 (segment (start 48.26 39.37) (end 52.07 39.37) (width 0.4) (layer B.Cu) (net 21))
 (segment (start 52.33 63.5) (end 49.53 63.5) (width 0.4) (layer B.Cu) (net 1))
 (segment (start 49.53 63.5) (end 48.26 64.77) (width 0.4) (layer B.Cu) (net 1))
 (segment (start 48.26 62.23) (end 49.53 60.96) (width 0.4) (layer B.Cu) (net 3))
 (segment (start 49.53 60.96) (end 52.33 60.96) (width 0.4) (layer B.Cu) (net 3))
 (segment (start 28.18384 36.87572) (end 32.97428 36.87572) (width 0.4) (layer B.Cu) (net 6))
 (segment (start 32.97428 36.87572) (end 33.02 36.83) (width 0.4) (layer B.Cu) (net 6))
 (segment (start 28.18384 39.41572) (end 32.97428 39.41572) (width 0.4) (layer B.Cu) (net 8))
 (segment (start 32.97428 39.41572) (end 33.02 39.37) (width 0.4) (layer B.Cu) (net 8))
 (segment (start 28.18384 41.95572) (end 32.97428 41.95572) (width 0.4) (layer B.Cu) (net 10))
 (segment (start 32.97428 41.95572) (end 33.02 41.91) (width 0.4) (layer B.Cu) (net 10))
 (segment (start 28.18384 44.49572) (end 32.97428 44.49572) (width 0.4) (layer B.Cu) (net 12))
 (segment (start 32.97428 44.49572) (end 33.02 44.45) (width 0.4) (layer B.Cu) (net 12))
 (segment (start 28.18384 47.03572) (end 32.97428 47.03572) (width 0.4) (layer B.Cu) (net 14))
 (segment (start 32.97428 47.03572) (end 33.02 46.99) (width 0.4) (layer B.Cu) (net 14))
 (segment (start 28.18384 49.57572) (end 32.97428 49.57572) (width 0.4) (layer B.Cu) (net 16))
 (segment (start 32.97428 49.57572) (end 33.02 49.53) (width 0.4) (layer B.Cu) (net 16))
 (segment (start 28.18384 52.11572) (end 32.97428 52.11572) (width 0.4) (layer B.Cu) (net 18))
 (segment (start 32.97428 52.11572) (end 33.02 52.07) (width 0.4) (layer B.Cu) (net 18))
 (segment (start 28.18384 54.65572) (end 32.97428 54.65572) (width 0.4) (layer B.Cu) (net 20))
 (segment (start 32.97428 54.65572) (end 33.02 54.61) (width 0.4) (layer B.Cu) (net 20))
 (segment (start 28.18384 59.73572) (end 32.97428 59.73572) (width 0.4) (layer B.Cu) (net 24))
 (segment (start 32.97428 59.73572) (end 33.02 59.69) (width 0.4) (layer B.Cu) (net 24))
 (segment (start 28.18384 64.81572) (end 32.97428 64.81572) (width 0.4) (layer B.Cu) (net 27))
 (segment (start 32.97428 64.81572) (end 33.02 64.77) (width 0.4) (layer B.Cu) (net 27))
 (segment (start 52.33 58.42) (end 49.53 58.42) (width 0.4) (layer B.Cu) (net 5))
 (segment (start 49.53 58.42) (end 48.26 59.69) (width 0.4) (layer B.Cu) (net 5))
 (segment (start 50.8 54.61) (end 52.07 55.88) (width 0.4) (layer B.Cu) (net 9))
 (segment (start 48.26 54.61) (end 50.8 54.61) (width 0.4) (layer B.Cu) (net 9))
 (segment (start 50.8 52.07) (end 52.07 53.34) (width 0.4) (layer B.Cu) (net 11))
 (segment (start 48.26 52.07) (end 50.8 52.07) (width 0.4) (layer B.Cu) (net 11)))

